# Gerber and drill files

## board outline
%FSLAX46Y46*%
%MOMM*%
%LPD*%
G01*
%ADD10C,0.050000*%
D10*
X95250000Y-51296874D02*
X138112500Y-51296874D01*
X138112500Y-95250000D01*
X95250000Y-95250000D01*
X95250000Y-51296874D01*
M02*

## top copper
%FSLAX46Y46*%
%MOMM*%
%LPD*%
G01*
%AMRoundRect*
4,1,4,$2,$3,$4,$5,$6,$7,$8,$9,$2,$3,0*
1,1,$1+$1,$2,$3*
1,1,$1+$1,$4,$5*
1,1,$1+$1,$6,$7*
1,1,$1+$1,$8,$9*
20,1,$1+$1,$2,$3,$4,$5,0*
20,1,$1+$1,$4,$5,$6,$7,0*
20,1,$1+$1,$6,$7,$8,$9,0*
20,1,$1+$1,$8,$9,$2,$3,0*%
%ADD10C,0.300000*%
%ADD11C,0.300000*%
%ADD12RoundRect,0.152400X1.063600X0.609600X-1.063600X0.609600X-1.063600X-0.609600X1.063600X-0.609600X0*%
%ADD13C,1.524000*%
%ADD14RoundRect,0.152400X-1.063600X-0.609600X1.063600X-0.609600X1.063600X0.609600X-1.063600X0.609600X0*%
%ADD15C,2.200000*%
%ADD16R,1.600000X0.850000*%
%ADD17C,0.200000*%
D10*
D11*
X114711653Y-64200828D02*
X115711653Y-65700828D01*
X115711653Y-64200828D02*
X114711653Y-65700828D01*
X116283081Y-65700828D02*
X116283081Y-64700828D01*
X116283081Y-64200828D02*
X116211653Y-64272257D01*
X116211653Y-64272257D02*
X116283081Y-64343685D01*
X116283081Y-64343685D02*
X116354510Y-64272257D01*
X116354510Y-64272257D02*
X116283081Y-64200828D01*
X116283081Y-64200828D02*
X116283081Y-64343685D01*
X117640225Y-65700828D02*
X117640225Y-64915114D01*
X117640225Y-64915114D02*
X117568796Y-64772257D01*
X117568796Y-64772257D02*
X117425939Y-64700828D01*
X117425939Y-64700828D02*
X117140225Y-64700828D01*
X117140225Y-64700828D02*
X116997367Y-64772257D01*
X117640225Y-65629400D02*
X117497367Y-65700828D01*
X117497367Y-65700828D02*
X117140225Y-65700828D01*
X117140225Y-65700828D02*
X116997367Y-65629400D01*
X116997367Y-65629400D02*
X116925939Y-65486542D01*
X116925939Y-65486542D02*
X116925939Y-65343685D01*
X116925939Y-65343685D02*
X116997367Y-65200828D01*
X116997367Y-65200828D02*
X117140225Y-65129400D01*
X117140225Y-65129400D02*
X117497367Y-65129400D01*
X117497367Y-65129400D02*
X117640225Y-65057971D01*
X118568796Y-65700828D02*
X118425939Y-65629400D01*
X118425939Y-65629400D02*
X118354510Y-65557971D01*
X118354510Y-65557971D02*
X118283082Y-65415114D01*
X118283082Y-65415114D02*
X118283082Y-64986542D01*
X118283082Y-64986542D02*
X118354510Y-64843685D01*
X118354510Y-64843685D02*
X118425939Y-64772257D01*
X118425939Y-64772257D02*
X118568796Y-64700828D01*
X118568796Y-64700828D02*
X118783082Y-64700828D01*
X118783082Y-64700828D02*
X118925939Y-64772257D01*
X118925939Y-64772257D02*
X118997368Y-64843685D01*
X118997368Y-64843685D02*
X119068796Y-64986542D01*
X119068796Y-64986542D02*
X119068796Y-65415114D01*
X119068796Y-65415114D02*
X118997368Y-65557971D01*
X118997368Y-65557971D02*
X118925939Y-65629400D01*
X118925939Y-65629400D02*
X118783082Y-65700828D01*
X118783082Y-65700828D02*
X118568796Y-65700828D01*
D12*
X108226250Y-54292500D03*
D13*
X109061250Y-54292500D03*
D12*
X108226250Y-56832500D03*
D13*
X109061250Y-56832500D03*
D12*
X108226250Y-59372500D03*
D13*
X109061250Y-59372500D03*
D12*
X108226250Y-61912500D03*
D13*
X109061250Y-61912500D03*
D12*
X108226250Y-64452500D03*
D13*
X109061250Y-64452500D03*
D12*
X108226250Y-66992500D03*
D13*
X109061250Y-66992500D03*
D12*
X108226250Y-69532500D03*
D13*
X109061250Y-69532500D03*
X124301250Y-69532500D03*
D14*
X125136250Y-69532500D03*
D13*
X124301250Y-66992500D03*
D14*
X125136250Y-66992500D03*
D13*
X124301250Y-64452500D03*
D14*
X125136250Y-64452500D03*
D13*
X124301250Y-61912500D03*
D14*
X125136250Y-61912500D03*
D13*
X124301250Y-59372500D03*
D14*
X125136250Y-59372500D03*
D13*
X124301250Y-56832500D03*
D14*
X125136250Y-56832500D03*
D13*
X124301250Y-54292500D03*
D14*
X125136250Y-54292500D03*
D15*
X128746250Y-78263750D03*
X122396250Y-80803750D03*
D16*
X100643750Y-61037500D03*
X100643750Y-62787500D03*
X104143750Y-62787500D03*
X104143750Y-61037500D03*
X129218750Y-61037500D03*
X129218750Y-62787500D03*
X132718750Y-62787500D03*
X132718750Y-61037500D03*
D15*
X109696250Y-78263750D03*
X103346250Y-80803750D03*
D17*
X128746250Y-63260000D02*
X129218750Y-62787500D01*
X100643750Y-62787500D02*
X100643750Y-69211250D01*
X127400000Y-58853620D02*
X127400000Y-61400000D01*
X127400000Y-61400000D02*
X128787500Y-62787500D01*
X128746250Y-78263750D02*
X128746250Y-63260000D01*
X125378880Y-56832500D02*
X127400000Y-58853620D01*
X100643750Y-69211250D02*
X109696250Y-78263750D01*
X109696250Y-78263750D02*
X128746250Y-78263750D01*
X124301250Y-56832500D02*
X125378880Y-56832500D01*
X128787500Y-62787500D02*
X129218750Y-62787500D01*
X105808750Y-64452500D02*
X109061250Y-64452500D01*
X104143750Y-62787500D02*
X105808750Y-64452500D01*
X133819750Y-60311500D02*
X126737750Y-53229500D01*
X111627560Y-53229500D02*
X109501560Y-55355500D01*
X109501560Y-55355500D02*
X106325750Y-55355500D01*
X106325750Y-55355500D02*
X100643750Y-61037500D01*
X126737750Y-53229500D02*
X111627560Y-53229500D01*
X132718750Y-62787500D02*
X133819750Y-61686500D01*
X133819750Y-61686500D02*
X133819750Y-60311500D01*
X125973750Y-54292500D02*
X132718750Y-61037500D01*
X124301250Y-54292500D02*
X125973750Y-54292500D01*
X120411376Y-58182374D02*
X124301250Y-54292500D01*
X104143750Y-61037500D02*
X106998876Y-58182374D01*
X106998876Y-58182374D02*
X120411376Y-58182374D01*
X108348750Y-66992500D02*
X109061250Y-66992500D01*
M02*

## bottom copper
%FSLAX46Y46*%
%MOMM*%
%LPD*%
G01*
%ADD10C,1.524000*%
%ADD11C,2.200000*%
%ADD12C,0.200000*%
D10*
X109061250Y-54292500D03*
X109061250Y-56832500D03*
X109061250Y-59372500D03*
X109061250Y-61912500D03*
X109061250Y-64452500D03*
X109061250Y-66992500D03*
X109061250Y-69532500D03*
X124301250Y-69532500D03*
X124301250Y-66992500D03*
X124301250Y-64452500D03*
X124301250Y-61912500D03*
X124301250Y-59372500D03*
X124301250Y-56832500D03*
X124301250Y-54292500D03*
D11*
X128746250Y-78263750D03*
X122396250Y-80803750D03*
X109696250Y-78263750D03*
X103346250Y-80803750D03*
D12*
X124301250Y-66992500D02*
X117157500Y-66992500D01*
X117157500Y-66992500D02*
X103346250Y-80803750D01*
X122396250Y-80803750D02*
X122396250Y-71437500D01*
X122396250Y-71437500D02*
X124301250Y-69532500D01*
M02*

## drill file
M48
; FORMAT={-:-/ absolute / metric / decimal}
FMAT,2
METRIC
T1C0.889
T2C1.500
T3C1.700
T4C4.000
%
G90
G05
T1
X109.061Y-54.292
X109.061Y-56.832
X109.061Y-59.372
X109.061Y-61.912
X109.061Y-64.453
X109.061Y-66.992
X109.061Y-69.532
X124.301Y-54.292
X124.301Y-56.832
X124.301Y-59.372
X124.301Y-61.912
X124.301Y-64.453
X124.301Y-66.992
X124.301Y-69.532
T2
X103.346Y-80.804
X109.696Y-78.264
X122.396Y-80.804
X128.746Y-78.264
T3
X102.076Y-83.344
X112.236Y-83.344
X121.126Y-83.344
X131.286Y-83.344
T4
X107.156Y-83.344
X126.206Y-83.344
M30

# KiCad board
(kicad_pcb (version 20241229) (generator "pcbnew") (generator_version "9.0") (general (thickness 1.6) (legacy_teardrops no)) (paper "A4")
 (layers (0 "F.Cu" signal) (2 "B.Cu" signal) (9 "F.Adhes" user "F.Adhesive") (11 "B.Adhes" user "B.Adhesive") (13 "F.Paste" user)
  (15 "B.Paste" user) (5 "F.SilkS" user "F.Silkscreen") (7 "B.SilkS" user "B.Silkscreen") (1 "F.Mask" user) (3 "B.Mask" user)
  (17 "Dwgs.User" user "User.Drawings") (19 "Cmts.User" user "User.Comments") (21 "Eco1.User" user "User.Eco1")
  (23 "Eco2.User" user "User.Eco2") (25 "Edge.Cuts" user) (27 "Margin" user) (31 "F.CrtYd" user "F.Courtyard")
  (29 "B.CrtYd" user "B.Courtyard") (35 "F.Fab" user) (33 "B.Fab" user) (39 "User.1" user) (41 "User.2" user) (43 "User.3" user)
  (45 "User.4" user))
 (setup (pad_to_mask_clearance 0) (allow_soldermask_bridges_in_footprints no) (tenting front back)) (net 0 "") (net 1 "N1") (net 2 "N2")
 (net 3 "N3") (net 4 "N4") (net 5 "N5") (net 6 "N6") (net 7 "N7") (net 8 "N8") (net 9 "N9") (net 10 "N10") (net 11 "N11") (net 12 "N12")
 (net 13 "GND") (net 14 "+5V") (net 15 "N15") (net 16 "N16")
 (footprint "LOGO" (layer "F.Cu") (at 99.4 55.6)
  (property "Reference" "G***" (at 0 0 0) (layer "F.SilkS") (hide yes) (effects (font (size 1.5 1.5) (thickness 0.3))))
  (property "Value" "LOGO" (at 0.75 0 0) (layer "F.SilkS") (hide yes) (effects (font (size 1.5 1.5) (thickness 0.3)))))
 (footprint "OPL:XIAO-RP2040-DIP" (layer "F.Cu") (at 116.68125 61.9125)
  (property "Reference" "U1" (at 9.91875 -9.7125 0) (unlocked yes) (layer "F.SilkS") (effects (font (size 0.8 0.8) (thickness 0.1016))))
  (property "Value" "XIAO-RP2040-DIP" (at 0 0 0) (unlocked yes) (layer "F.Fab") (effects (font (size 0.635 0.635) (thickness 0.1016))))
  (pad "1" smd roundrect (at -8.455 -7.62 180) (size 2.432 1.524) (layers "F.Cu" "F.Mask") (roundrect_rratio 0.1) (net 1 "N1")
   (thermal_bridge_angle 45))
  (pad "1" thru_hole circle (at -7.62 -7.62 180) (size 1.524 1.524) (drill 0.889) (layers "*.Cu" "*.Mask") (remove_unused_layers no)
   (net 1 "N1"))
  (pad "2" smd roundrect (at -8.455 -5.08 180) (size 2.432 1.524) (layers "F.Cu" "F.Mask") (roundrect_rratio 0.1) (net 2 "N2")
   (thermal_bridge_angle 45))
  (pad "2" thru_hole circle (at -7.62 -5.08 180) (size 1.524 1.524) (drill 0.889) (layers "*.Cu" "*.Mask") (remove_unused_layers no)
   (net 2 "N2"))
  (pad "3" smd roundrect (at -8.455 -2.54 180) (size 2.432 1.524) (layers "F.Cu" "F.Mask") (roundrect_rratio 0.1) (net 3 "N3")
   (thermal_bridge_angle 45))
  (pad "3" thru_hole circle (at -7.62 -2.54 180) (size 1.524 1.524) (drill 0.889) (layers "*.Cu" "*.Mask") (remove_unused_layers no)
   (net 3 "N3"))
  (pad "4" smd roundrect (at -8.455 0 180) (size 2.432 1.524) (layers "F.Cu" "F.Mask") (roundrect_rratio 0.1) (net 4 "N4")
   (thermal_bridge_angle 45))
  (pad "4" thru_hole circle (at -7.62 0 180) (size 1.524 1.524) (drill 0.889) (layers "*.Cu" "*.Mask") (remove_unused_layers no)
   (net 4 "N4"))
  (pad "5" smd roundrect (at -8.455 2.54 180) (size 2.432 1.524) (layers "F.Cu" "F.Mask") (roundrect_rratio 0.1) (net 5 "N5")
   (thermal_bridge_angle 45))
  (pad "5" thru_hole circle (at -7.62 2.54 180) (size 1.524 1.524) (drill 0.889) (layers "*.Cu" "*.Mask") (remove_unused_layers no)
   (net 5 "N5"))
  (pad "6" smd roundrect (at -8.455 5.08 180) (size 2.432 1.524) (layers "F.Cu" "F.Mask") (roundrect_rratio 0.1) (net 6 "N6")
   (thermal_bridge_angle 45))
  (pad "6" thru_hole circle (at -7.62 5.08 180) (size 1.524 1.524) (drill 0.889) (layers "*.Cu" "*.Mask") (remove_unused_layers no)
   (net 6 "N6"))
  (pad "7" smd roundrect (at -8.455 7.62 180) (size 2.432 1.524) (layers "F.Cu" "F.Mask") (roundrect_rratio 0.1) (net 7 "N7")
   (thermal_bridge_angle 45))
  (pad "7" thru_hole circle (at -7.62 7.62 180) (size 1.524 1.524) (drill 0.889) (layers "*.Cu" "*.Mask") (remove_unused_layers no)
   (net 7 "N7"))
  (pad "8" thru_hole circle (at 7.62 7.62) (size 1.524 1.524) (drill 0.889) (layers "*.Cu" "*.Mask") (remove_unused_layers no) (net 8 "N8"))
  (pad "8" smd roundrect (at 8.455 7.62) (size 2.432 1.524) (layers "F.Cu" "F.Mask") (roundrect_rratio 0.1) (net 8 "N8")
   (thermal_bridge_angle 45))
  (pad "9" thru_hole circle (at 7.62 5.08) (size 1.524 1.524) (drill 0.889) (layers "*.Cu" "*.Mask") (remove_unused_layers no) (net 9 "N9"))
  (pad "9" smd roundrect (at 8.455 5.08) (size 2.432 1.524) (layers "F.Cu" "F.Mask") (roundrect_rratio 0.1) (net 9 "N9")
   (thermal_bridge_angle 45))
  (pad "10" thru_hole circle (at 7.62 2.54) (size 1.524 1.524) (drill 0.889) (layers "*.Cu" "*.Mask") (remove_unused_layers no)
   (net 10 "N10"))
  (pad "10" smd roundrect (at 8.455 2.54) (size 2.432 1.524) (layers "F.Cu" "F.Mask") (roundrect_rratio 0.1) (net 10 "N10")
   (thermal_bridge_angle 45))
  (pad "11" thru_hole circle (at 7.62 0) (size 1.524 1.524) (drill 0.889) (layers "*.Cu" "*.Mask") (remove_unused_layers no) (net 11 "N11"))
  (pad "11" smd roundrect (at 8.455 0) (size 2.432 1.524) (layers "F.Cu" "F.Mask") (roundrect_rratio 0.1) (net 11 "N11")
   (thermal_bridge_angle 45))
  (pad "12" thru_hole circle (at 7.62 -2.54) (size 1.524 1.524) (drill 0.889) (layers "*.Cu" "*.Mask") (remove_unused_layers no)
   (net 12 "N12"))
  (pad "12" smd roundrect (at 8.455 -2.54) (size 2.432 1.524) (layers "F.Cu" "F.Mask") (roundrect_rratio 0.1) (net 12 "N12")
   (thermal_bridge_angle 45))
  (pad "13" thru_hole circle (at 7.62 -5.08) (size 1.524 1.524) (drill 0.889) (layers "*.Cu" "*.Mask") (remove_unused_layers no)
   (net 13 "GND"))
  (pad "13" smd roundrect (at 8.455 -5.08) (size 2.432 1.524) (layers "F.Cu" "F.Mask") (roundrect_rratio 0.1) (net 13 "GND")
   (thermal_bridge_angle 45))
  (pad "14" thru_hole circle (at 7.62 -7.62) (size 1.524 1.524) (drill 0.889) (layers "*.Cu" "*.Mask") (remove_unused_layers no)
   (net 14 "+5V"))
  (pad "14" smd roundrect (at 8.455 -7.62) (size 2.432 1.524) (layers "F.Cu" "F.Mask") (roundrect_rratio 0.1) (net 14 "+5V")
   (thermal_bridge_angle 45)))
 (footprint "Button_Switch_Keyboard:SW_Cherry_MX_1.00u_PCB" (layer "F.Cu") (at 128.74625 78.26375)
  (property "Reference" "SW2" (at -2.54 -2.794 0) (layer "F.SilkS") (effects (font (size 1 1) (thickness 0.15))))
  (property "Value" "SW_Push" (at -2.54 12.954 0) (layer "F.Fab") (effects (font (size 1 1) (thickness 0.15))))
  (pad "" np_thru_hole circle (at -7.62 5.08) (size 1.7 1.7) (drill 1.7) (layers "*.Cu" "*.Mask"))
  (pad "" np_thru_hole circle (at -2.54 5.08) (size 4 4) (drill 4) (layers "*.Cu" "*.Mask"))
  (pad "" np_thru_hole circle (at 2.54 5.08) (size 1.7 1.7) (drill 1.7) (layers "*.Cu" "*.Mask"))
  (pad "1" thru_hole circle (at 0 0) (size 2.2 2.2) (drill 1.5) (layers "*.Cu" "*.Mask") (remove_unused_layers no) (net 13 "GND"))
  (pad "2" thru_hole circle (at -6.35 2.54) (size 2.2 2.2) (drill 1.5) (layers "*.Cu" "*.Mask") (remove_unused_layers no) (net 8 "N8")))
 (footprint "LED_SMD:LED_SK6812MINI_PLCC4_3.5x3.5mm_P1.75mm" (layer "F.Cu") (at 102.39375 61.9125)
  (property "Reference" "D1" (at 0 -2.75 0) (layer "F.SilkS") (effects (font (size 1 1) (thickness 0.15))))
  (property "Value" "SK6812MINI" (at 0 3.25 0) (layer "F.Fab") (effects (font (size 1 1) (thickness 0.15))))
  (pad "1" smd rect (at -1.75 -0.875) (size 1.6 0.85) (layers "F.Cu" "F.Mask" "F.Paste") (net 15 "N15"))
  (pad "2" smd rect (at -1.75 0.875) (size 1.6 0.85) (layers "F.Cu" "F.Mask" "F.Paste") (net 13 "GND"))
  (pad "3" smd rect (at 1.75 0.875) (size 1.6 0.85) (layers "F.Cu" "F.Mask" "F.Paste") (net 5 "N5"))
  (pad "4" smd rect (at 1.75 -0.875) (size 1.6 0.85) (layers "F.Cu" "F.Mask" "F.Paste") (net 14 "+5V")))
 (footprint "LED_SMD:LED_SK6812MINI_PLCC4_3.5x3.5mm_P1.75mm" (layer "F.Cu") (at 130.96875 61.9125)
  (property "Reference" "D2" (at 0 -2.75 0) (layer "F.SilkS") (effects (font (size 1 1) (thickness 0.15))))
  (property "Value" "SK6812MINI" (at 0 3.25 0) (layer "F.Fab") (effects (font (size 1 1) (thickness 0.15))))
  (pad "1" smd rect (at -1.75 -0.875) (size 1.6 0.85) (layers "F.Cu" "F.Mask" "F.Paste") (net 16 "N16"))
  (pad "2" smd rect (at -1.75 0.875) (size 1.6 0.85) (layers "F.Cu" "F.Mask" "F.Paste") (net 13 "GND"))
  (pad "3" smd rect (at 1.75 0.875) (size 1.6 0.85) (layers "F.Cu" "F.Mask" "F.Paste") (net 15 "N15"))
  (pad "4" smd rect (at 1.75 -0.875) (size 1.6 0.85) (layers "F.Cu" "F.Mask" "F.Paste") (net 14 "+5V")))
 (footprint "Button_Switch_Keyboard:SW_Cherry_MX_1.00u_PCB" (layer "F.Cu") (at 109.69625 78.26375)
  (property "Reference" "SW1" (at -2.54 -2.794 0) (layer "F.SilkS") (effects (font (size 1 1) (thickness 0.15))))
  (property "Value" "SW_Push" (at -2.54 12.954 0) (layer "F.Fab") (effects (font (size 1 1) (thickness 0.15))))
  (pad "" np_thru_hole circle (at -7.62 5.08) (size 1.7 1.7) (drill 1.7) (layers "*.Cu" "*.Mask"))
  (pad "" np_thru_hole circle (at -2.54 5.08) (size 4 4) (drill 4) (layers "*.Cu" "*.Mask"))
  (pad "" np_thru_hole circle (at 2.54 5.08) (size 1.7 1.7) (drill 1.7) (layers "*.Cu" "*.Mask"))
  (pad "1" thru_hole circle (at 0 0) (size 2.2 2.2) (drill 1.5) (layers "*.Cu" "*.Mask") (remove_unused_layers no) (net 13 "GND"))
  (pad "2" thru_hole circle (at -6.35 2.54) (size 2.2 2.2) (drill 1.5) (layers "*.Cu" "*.Mask") (remove_unused_layers no) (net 9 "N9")))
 (gr_rect (start 95.25 51.296874) (end 138.1125 95.25) (stroke (width 0.05) (type default)) (fill no) (layer "Edge.Cuts"))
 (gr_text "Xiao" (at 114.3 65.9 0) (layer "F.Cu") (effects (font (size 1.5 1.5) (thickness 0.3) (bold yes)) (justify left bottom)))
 (segment (start 128.74625 63.26) (end 129.21875 62.7875) (width 0.2) (layer "F.Cu") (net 13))
 (segment (start 100.64375 62.7875) (end 100.64375 69.21125) (width 0.2) (layer "F.Cu") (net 13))
 (segment (start 127.4 58.85362) (end 127.4 61.4) (width 0.2) (layer "F.Cu") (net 13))
 (segment (start 127.4 61.4) (end 128.7875 62.7875) (width 0.2) (layer "F.Cu") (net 13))
 (segment (start 128.74625 78.26375) (end 128.74625 63.26) (width 0.2) (layer "F.Cu") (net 13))
 (segment (start 125.37888 56.8325) (end 127.4 58.85362) (width 0.2) (layer "F.Cu") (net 13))
 (segment (start 100.64375 69.21125) (end 109.69625 78.26375) (width 0.2) (layer "F.Cu") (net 13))
 (segment (start 109.69625 78.26375) (end 128.74625 78.26375) (width 0.2) (layer "F.Cu") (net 13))
 (segment (start 124.30125 56.8325) (end 125.37888 56.8325) (width 0.2) (layer "F.Cu") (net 13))
 (segment (start 128.7875 62.7875) (end 129.21875 62.7875) (width 0.2) (layer "F.Cu") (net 13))
 (segment (start 105.80875 64.4525) (end 109.06125 64.4525) (width 0.2) (layer "F.Cu") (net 5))
 (segment (start 104.14375 62.7875) (end 105.80875 64.4525) (width 0.2) (layer "F.Cu") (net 5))
 (segment (start 133.81975 60.3115) (end 126.73775 53.2295) (width 0.2) (layer "F.Cu") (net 15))
 (segment (start 111.62756 53.2295) (end 109.50156 55.3555) (width 0.2) (layer "F.Cu") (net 15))
 (segment (start 109.50156 55.3555) (end 106.32575 55.3555) (width 0.2) (layer "F.Cu") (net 15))
 (segment (start 106.32575 55.3555) (end 100.64375 61.0375) (width 0.2) (layer "F.Cu") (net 15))
 (segment (start 126.73775 53.2295) (end 111.62756 53.2295) (width 0.2) (layer "F.Cu") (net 15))
 (segment (start 132.71875 62.7875) (end 133.81975 61.6865) (width 0.2) (layer "F.Cu") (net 15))
 (segment (start 133.81975 61.6865) (end 133.81975 60.3115) (width 0.2) (layer "F.Cu") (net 15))
 (segment (start 125.97375 54.2925) (end 132.71875 61.0375) (width 0.2) (layer "F.Cu") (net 14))
 (segment (start 124.30125 54.2925) (end 125.97375 54.2925) (width 0.2) (layer "F.Cu") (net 14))
 (segment (start 120.411376 58.182374) (end 124.30125 54.2925) (width 0.2) (layer "F.Cu") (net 14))
 (segment (start 104.14375 61.0375) (end 106.998876 58.182374) (width 0.2) (layer "F.Cu") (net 14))
 (segment (start 106.998876 58.182374) (end 120.411376 58.182374) (width 0.2) (layer "F.Cu") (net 14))
 (segment (start 124.30125 66.9925) (end 117.1575 66.9925) (width 0.2) (layer "B.Cu") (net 9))
 (segment (start 117.1575 66.9925) (end 103.34625 80.80375) (width 0.2) (layer "B.Cu") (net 9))
 (segment (start 122.39625 80.80375) (end 122.39625 71.4375) (width 0.2) (layer "B.Cu") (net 8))
 (segment (start 122.39625 71.4375) (end 124.30125 69.5325) (width 0.2) (layer "B.Cu") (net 8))
 (segment (start 108.34875 66.9925) (end 109.06125 66.9925) (width 0.2) (layer "F.Cu") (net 6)))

